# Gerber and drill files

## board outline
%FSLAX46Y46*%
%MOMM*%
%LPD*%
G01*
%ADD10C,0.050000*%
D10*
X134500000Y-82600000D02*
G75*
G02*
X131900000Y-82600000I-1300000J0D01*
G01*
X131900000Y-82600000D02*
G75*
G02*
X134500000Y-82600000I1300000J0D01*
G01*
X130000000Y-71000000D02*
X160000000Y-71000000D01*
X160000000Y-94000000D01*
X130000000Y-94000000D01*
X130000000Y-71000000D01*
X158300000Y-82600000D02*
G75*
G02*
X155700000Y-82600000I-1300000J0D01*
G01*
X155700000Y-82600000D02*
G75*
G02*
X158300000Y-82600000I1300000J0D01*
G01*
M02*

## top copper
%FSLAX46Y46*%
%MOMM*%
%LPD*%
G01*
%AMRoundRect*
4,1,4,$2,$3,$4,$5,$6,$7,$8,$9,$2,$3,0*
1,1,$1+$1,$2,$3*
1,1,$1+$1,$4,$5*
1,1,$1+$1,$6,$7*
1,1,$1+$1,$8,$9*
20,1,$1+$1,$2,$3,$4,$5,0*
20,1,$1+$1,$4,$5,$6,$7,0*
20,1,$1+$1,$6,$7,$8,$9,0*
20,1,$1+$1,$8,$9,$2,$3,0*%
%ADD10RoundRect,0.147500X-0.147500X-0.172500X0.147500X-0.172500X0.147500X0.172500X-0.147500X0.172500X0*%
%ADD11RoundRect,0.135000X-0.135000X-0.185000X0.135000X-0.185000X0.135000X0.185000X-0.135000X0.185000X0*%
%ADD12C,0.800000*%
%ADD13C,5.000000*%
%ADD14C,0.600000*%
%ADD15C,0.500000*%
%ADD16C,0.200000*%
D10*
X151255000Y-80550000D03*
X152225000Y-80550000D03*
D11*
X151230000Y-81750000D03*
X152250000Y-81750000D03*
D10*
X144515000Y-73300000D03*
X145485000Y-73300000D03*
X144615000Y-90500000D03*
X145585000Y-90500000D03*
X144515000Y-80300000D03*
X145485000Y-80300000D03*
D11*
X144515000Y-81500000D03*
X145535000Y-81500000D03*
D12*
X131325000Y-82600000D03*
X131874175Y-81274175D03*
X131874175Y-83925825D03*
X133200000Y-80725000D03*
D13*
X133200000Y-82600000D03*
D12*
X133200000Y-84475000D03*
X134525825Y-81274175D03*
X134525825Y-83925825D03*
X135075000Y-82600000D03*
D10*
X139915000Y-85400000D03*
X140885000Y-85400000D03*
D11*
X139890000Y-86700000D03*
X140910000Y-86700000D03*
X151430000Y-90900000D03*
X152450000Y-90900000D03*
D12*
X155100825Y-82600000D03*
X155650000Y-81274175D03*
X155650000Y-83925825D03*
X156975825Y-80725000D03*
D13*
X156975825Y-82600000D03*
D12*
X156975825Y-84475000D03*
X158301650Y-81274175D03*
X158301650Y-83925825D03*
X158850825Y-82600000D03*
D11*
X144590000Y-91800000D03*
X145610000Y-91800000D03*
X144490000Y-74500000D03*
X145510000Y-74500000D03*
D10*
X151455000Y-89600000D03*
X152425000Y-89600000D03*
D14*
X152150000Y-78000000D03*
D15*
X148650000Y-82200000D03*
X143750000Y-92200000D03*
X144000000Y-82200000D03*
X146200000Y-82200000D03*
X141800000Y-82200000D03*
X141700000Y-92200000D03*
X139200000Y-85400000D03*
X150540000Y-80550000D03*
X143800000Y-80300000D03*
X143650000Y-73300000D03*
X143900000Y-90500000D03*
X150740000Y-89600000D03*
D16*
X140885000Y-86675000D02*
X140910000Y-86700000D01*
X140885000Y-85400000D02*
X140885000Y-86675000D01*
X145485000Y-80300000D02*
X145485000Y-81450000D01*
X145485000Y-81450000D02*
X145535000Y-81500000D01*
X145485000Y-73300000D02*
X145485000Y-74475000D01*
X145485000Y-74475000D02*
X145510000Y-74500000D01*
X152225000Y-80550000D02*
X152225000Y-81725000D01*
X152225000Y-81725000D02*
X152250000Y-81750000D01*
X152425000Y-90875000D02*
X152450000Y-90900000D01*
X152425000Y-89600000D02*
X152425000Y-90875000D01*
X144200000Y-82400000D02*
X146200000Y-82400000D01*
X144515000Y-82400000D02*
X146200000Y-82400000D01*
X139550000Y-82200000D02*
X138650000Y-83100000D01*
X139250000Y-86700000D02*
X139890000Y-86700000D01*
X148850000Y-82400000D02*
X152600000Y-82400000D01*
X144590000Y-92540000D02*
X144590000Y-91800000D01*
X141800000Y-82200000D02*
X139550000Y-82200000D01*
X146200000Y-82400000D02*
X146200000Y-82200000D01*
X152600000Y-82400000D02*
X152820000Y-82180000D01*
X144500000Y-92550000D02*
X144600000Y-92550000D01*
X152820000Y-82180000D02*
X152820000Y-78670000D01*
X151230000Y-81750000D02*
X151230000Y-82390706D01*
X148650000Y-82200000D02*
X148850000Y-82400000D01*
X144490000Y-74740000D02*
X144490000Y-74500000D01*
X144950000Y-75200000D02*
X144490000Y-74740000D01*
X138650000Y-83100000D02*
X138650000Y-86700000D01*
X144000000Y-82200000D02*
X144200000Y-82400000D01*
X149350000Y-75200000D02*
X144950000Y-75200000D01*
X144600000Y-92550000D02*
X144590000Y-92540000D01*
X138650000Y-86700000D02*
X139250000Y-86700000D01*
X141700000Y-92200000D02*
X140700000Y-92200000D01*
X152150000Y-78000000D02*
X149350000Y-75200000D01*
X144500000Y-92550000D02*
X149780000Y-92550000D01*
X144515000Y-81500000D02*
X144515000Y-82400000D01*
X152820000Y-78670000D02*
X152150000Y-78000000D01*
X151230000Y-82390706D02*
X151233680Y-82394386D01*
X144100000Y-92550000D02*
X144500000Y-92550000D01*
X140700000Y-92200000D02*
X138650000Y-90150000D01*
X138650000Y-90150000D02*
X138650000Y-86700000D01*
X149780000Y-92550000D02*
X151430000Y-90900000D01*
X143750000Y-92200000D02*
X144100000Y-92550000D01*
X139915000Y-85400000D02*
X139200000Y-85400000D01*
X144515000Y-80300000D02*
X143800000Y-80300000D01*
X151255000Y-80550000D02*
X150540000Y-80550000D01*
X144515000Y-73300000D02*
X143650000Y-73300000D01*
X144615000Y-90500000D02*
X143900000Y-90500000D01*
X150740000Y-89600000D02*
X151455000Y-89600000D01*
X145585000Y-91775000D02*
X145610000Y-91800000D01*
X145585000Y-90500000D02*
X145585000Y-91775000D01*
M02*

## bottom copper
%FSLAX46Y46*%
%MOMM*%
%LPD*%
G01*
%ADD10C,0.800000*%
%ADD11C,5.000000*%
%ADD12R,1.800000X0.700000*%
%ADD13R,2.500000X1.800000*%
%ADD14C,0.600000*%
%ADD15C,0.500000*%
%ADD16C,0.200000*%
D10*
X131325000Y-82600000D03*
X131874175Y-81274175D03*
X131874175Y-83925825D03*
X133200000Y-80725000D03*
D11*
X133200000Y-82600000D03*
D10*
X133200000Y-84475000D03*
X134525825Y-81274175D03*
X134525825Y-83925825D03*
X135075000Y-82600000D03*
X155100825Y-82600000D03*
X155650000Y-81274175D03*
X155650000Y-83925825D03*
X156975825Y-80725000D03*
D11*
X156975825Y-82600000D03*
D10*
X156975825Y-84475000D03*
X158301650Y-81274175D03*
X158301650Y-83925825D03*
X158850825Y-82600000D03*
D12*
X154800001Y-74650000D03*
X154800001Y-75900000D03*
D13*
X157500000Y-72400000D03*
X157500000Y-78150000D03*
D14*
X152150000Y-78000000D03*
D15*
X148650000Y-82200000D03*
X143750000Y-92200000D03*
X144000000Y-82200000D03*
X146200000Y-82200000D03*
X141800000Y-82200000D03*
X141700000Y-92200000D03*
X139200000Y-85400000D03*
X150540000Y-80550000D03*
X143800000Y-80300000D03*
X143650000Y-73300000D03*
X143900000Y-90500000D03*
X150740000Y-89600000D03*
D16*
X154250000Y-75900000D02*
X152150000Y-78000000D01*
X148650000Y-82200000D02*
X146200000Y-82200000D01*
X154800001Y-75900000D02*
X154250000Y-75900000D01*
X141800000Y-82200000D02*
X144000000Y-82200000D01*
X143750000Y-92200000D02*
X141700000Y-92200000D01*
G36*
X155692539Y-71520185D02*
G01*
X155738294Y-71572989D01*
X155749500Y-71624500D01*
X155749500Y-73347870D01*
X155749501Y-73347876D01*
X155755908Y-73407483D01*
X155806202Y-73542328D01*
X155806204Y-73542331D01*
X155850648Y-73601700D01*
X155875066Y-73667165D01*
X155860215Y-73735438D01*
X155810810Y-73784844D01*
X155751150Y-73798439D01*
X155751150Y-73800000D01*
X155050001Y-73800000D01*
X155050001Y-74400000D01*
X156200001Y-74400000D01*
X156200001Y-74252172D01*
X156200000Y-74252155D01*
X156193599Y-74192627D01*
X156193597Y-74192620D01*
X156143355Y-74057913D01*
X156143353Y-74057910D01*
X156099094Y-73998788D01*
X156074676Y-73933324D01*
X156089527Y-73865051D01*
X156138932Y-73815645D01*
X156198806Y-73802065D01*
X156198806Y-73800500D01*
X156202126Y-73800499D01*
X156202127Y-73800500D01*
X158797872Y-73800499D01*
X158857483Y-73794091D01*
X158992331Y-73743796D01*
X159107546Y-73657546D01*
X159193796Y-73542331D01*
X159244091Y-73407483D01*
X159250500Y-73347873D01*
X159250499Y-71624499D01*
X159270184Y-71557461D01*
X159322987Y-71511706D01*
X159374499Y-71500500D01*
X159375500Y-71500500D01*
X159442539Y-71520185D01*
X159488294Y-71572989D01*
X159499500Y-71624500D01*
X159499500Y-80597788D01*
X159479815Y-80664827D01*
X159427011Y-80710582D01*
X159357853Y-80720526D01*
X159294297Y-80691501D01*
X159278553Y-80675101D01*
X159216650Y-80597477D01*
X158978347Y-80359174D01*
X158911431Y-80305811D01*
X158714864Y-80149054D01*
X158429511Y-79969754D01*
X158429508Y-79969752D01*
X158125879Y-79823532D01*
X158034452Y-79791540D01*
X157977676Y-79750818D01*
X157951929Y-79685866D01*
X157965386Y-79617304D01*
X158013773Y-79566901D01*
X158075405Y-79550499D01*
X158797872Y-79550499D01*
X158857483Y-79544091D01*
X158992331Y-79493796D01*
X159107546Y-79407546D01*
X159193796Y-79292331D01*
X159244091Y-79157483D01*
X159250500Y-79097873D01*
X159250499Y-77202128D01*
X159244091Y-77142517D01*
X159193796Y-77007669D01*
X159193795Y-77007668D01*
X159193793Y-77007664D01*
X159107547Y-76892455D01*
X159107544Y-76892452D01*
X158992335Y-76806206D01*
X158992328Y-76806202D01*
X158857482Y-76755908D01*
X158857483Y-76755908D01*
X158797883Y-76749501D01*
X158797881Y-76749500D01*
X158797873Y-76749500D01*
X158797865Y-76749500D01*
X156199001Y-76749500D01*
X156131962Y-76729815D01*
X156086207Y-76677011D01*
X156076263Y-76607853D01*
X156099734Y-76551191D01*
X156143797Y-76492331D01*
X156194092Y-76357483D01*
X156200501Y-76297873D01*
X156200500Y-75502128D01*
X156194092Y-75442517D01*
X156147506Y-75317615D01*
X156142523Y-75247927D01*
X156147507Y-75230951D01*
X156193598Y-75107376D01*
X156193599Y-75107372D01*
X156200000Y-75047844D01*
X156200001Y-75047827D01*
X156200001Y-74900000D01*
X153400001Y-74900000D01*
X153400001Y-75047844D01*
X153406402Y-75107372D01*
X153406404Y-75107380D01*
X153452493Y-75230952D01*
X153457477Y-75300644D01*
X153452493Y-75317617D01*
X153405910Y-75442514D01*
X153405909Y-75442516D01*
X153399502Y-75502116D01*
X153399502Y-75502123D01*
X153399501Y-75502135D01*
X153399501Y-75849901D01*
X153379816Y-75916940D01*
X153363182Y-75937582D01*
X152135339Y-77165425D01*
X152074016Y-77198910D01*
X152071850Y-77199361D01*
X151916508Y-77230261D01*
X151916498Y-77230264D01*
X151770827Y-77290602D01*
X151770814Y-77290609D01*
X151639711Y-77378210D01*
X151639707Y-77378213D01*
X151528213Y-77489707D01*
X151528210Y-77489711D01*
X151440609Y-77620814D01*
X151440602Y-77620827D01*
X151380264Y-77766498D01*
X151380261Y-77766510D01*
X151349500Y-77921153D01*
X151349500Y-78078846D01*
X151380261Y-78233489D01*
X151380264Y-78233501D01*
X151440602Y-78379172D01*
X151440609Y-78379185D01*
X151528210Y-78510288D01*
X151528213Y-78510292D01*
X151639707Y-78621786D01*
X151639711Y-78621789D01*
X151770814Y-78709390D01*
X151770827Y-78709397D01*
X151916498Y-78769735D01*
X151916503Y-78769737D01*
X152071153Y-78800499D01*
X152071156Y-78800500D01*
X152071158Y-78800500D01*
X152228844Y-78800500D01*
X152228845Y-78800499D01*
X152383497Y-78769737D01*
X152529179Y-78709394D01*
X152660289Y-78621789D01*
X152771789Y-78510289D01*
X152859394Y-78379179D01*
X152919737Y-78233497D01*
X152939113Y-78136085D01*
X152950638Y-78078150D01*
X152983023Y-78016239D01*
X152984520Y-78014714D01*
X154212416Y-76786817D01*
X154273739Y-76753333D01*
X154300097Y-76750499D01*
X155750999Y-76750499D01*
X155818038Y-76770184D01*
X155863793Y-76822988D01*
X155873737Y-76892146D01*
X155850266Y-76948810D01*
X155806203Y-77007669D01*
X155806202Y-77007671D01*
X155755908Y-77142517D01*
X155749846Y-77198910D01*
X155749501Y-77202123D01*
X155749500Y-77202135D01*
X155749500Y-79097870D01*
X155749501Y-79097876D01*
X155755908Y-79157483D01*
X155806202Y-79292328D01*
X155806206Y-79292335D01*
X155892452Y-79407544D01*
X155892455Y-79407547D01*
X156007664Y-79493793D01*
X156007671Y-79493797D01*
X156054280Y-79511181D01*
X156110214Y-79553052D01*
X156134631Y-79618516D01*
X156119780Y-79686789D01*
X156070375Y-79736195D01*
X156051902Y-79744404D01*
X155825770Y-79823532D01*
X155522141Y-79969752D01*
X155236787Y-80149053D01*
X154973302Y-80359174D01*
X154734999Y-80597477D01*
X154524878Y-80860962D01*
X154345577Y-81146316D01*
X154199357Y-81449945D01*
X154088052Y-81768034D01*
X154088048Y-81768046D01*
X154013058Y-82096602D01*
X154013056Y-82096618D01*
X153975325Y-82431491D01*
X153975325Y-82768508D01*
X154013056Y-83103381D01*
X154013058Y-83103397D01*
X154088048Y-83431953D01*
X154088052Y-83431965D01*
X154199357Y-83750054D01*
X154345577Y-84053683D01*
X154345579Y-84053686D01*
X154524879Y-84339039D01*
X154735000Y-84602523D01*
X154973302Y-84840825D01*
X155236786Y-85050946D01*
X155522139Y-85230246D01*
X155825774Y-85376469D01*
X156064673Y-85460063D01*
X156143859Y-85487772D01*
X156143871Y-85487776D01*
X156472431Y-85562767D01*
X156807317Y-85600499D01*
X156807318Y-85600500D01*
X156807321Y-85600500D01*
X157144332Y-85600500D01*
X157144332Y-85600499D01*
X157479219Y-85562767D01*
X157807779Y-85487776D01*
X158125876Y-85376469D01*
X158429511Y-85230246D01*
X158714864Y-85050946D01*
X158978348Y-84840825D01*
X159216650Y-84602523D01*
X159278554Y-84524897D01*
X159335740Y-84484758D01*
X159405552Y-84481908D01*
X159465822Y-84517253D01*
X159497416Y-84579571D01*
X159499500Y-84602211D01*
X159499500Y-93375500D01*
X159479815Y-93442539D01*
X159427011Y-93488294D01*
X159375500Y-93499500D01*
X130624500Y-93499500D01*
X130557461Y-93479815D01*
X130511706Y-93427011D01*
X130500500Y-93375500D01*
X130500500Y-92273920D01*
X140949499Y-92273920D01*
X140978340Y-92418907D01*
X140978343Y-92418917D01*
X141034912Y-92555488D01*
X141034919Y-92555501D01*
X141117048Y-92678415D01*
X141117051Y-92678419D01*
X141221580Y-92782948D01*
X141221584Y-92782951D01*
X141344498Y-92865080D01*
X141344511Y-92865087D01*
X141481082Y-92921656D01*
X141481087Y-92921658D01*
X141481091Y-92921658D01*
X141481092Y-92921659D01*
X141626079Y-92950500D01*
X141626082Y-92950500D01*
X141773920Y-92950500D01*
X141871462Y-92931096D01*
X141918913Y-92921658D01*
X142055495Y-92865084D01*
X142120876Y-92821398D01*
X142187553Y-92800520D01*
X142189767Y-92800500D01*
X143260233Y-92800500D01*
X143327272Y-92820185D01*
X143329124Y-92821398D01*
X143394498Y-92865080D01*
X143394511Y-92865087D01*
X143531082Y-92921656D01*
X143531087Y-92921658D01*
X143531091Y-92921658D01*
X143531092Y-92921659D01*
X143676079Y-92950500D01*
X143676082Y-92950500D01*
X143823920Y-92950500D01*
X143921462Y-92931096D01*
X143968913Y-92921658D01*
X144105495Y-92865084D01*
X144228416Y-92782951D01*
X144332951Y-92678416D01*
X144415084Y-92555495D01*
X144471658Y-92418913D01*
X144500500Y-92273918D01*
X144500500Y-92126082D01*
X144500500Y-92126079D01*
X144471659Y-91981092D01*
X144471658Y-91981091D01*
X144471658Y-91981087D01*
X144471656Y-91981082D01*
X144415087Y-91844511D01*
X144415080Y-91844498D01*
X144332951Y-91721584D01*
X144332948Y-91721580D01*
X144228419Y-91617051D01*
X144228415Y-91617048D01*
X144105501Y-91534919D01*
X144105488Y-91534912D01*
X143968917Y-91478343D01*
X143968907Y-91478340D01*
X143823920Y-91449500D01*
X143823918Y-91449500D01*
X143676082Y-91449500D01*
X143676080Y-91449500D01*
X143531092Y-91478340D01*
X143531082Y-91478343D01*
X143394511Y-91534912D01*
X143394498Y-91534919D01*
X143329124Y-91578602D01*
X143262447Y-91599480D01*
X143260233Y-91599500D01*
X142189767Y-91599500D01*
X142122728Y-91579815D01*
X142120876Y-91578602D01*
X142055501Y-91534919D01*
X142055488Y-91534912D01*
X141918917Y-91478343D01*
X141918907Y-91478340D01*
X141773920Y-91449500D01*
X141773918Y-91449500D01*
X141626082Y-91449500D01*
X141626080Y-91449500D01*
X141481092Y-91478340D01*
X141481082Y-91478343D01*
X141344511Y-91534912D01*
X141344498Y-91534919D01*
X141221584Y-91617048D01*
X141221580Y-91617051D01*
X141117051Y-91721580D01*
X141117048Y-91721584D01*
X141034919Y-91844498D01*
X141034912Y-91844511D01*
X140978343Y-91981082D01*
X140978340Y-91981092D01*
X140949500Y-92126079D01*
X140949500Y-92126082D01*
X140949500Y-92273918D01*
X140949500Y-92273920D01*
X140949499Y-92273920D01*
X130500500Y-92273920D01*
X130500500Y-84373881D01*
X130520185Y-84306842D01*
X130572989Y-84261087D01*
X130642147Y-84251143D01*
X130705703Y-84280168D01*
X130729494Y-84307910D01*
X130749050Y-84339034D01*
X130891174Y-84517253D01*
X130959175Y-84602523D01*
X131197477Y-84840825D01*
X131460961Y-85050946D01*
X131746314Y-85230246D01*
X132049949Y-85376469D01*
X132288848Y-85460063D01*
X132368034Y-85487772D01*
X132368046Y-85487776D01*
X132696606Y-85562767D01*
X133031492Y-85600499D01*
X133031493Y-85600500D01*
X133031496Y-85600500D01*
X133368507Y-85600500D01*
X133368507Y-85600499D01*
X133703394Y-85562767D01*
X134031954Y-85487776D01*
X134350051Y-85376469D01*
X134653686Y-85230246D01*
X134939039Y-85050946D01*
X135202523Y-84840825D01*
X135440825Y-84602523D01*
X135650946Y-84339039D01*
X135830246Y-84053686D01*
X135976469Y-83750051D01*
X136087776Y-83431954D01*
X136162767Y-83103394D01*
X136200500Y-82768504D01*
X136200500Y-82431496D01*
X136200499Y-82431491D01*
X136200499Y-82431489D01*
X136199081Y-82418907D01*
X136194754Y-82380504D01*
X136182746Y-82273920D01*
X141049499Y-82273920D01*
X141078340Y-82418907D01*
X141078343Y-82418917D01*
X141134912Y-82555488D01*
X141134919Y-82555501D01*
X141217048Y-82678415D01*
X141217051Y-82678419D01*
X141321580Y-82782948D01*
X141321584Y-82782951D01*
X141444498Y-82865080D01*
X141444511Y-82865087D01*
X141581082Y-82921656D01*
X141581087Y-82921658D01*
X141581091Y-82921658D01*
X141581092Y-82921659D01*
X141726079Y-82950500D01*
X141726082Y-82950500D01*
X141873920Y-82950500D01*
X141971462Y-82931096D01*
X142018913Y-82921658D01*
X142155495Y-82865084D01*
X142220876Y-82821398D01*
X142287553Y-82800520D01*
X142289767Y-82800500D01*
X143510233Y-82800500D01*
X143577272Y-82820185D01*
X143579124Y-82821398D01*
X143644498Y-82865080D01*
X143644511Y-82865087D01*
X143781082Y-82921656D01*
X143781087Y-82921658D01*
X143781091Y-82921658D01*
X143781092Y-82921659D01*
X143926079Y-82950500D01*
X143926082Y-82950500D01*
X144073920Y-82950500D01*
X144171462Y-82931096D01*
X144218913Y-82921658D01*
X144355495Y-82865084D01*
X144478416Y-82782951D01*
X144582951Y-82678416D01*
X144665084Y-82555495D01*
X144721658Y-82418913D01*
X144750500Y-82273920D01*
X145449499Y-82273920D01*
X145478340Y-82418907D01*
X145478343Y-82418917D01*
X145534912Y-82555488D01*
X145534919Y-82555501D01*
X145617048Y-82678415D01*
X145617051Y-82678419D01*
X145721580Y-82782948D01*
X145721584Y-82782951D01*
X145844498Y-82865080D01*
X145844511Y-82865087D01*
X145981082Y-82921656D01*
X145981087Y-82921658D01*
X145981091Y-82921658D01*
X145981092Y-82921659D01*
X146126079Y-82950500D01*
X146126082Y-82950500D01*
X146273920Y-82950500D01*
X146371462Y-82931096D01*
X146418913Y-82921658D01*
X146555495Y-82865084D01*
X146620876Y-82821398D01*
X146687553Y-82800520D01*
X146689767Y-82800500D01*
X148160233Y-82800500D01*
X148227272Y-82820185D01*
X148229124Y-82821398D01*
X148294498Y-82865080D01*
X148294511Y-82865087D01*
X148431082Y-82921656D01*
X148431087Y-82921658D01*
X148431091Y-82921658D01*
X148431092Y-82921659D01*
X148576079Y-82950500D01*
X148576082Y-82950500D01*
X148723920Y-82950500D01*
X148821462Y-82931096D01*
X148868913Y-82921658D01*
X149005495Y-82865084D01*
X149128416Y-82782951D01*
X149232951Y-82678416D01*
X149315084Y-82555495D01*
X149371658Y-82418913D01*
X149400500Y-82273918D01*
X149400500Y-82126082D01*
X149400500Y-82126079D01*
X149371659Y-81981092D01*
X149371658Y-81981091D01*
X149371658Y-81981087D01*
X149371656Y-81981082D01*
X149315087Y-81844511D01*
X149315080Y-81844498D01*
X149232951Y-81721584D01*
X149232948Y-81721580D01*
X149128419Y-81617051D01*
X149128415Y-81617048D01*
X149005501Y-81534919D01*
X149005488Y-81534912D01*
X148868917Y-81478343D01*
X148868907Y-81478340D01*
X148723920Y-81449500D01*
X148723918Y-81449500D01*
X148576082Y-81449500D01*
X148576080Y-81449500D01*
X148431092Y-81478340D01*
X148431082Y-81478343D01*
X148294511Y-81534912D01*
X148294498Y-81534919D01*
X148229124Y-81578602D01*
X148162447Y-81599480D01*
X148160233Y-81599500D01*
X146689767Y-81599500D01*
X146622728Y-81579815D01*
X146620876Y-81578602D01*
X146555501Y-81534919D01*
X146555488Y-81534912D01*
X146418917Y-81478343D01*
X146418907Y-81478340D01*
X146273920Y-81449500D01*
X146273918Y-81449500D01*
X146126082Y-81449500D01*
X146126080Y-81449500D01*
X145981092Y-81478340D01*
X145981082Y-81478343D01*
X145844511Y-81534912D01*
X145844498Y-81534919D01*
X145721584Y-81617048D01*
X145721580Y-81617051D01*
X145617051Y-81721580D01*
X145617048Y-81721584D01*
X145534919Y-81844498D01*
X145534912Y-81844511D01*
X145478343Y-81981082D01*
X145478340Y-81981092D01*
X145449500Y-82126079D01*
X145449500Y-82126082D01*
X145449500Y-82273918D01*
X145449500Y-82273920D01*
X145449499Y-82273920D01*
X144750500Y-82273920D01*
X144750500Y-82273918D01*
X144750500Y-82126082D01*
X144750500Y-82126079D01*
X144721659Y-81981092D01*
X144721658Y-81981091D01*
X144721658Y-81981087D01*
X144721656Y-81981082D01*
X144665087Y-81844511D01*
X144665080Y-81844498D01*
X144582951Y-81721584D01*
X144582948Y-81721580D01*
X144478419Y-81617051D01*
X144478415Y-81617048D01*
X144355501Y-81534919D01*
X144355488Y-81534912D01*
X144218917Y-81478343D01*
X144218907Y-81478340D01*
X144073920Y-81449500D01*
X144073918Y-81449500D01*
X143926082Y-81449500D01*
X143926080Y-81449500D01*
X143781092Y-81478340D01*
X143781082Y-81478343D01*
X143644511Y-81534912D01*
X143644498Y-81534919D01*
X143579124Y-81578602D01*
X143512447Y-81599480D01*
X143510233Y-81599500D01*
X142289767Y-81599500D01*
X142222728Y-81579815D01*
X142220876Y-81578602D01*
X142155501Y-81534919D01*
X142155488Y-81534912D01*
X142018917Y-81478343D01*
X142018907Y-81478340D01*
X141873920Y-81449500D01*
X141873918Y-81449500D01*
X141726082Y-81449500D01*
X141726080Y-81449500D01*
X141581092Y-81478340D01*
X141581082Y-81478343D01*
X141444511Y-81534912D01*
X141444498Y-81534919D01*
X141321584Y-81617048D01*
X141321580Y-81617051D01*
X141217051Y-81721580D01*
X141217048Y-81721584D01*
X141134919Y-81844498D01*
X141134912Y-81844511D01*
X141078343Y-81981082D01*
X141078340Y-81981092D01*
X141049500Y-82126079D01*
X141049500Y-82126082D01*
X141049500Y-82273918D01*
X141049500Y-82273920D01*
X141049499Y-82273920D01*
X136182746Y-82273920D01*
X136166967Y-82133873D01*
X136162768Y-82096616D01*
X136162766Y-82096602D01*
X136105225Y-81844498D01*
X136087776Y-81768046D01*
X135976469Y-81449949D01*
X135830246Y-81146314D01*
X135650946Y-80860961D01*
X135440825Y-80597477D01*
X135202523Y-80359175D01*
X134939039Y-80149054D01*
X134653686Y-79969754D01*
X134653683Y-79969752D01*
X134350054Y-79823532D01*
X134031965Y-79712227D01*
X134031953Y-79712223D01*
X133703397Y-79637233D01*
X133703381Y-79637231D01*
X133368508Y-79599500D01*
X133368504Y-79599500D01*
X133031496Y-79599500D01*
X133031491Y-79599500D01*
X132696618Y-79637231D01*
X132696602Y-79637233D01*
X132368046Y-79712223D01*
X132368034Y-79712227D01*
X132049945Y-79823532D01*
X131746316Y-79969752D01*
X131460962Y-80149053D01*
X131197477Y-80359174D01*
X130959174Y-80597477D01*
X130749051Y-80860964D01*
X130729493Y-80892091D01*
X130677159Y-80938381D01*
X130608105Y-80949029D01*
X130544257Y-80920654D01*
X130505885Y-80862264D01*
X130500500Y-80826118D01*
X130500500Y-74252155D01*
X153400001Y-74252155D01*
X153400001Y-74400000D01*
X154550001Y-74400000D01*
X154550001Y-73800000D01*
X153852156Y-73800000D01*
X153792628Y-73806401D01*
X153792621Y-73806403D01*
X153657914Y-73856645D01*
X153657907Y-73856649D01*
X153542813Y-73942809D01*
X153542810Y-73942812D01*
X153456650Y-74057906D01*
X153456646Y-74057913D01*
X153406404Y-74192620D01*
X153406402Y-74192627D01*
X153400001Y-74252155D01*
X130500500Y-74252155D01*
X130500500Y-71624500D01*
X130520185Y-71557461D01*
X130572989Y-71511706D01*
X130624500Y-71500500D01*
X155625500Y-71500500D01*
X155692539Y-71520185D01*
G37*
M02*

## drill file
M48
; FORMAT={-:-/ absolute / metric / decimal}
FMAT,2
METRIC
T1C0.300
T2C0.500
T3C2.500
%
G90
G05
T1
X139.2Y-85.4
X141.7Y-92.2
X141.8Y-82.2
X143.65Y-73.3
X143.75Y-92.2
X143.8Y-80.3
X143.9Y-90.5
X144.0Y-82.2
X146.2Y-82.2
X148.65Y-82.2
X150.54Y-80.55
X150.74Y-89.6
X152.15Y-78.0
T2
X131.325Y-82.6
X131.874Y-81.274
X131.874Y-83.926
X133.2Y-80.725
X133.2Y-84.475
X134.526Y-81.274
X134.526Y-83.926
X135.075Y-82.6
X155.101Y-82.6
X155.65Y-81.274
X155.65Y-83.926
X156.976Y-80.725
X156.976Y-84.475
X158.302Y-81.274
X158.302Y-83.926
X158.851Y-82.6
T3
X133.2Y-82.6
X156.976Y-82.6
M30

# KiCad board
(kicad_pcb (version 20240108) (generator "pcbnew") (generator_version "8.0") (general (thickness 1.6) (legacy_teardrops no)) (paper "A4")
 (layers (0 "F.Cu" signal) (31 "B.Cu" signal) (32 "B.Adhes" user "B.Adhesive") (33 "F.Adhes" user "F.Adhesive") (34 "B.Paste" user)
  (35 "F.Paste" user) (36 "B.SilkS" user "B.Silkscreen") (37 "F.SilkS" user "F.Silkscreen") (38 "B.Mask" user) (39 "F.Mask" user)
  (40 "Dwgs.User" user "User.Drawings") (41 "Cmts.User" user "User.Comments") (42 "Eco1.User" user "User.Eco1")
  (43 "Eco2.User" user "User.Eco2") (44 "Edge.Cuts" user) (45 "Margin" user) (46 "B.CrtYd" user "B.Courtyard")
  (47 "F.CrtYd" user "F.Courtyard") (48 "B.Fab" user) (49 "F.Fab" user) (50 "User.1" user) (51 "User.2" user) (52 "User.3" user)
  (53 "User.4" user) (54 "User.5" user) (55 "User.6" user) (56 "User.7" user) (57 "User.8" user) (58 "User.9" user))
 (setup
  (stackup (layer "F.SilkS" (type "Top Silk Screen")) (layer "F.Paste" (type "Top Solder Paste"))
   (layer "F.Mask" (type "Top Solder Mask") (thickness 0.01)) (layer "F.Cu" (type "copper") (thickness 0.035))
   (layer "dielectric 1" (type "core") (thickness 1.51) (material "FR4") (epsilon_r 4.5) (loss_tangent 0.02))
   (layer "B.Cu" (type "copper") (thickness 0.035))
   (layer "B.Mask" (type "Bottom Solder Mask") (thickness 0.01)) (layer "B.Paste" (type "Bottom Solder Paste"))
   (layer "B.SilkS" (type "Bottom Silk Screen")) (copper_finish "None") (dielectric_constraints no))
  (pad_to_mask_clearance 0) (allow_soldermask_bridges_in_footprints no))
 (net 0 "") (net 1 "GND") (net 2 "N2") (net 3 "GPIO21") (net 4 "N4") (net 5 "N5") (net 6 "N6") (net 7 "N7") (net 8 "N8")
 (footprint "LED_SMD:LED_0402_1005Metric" (layer "F.Cu") (at 151.74 80.55)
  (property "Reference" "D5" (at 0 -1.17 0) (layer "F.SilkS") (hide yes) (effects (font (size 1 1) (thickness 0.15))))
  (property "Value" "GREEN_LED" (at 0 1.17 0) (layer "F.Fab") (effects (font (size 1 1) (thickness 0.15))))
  (pad "1" smd roundrect (at -0.485 0) (size 0.59 0.64) (layers "F.Cu" "F.Paste" "F.Mask") (roundrect_rratio 0.25) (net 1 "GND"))
  (pad "2" smd roundrect (at 0.485 0) (size 0.59 0.64) (layers "F.Cu" "F.Paste" "F.Mask") (roundrect_rratio 0.25) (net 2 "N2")))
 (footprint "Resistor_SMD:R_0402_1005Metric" (layer "F.Cu") (at 151.74 81.75)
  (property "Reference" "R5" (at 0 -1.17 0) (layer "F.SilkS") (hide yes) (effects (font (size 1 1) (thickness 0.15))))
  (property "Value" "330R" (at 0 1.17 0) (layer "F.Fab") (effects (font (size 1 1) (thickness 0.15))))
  (pad "1" smd roundrect (at -0.51 0) (size 0.54 0.64) (layers "F.Cu" "F.Paste" "F.Mask") (roundrect_rratio 0.25) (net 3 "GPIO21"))
  (pad "2" smd roundrect (at 0.51 0) (size 0.54 0.64) (layers "F.Cu" "F.Paste" "F.Mask") (roundrect_rratio 0.25) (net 2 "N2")))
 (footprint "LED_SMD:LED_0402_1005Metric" (layer "F.Cu") (at 145 73.3)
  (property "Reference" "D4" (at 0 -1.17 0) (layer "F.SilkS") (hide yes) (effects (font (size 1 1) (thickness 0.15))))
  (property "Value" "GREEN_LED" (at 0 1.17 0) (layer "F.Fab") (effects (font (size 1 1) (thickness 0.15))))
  (pad "1" smd roundrect (at -0.485 0) (size 0.59 0.64) (layers "F.Cu" "F.Paste" "F.Mask") (roundrect_rratio 0.25) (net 1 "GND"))
  (pad "2" smd roundrect (at 0.485 0) (size 0.59 0.64) (layers "F.Cu" "F.Paste" "F.Mask") (roundrect_rratio 0.25) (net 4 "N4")))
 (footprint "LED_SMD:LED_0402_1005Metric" (layer "F.Cu") (at 145.1 90.5)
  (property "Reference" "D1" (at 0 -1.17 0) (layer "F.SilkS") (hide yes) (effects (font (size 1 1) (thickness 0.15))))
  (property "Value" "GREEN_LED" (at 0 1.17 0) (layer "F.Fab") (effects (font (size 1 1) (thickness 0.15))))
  (pad "1" smd roundrect (at -0.485 0) (size 0.59 0.64) (layers "F.Cu" "F.Paste" "F.Mask") (roundrect_rratio 0.25) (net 1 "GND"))
  (pad "2" smd roundrect (at 0.485 0) (size 0.59 0.64) (layers "F.Cu" "F.Paste" "F.Mask") (roundrect_rratio 0.25) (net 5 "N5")))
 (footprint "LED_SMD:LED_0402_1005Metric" (layer "F.Cu") (at 145 80.3)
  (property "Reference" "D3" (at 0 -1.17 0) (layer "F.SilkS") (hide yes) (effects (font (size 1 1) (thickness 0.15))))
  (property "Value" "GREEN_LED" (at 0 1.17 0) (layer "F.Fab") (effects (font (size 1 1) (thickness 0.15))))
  (pad "1" smd roundrect (at -0.485 0) (size 0.59 0.64) (layers "F.Cu" "F.Paste" "F.Mask") (roundrect_rratio 0.25) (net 1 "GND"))
  (pad "2" smd roundrect (at 0.485 0) (size 0.59 0.64) (layers "F.Cu" "F.Paste" "F.Mask") (roundrect_rratio 0.25) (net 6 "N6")))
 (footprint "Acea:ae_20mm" (layer "F.Cu") (at 144.822605 82.737829)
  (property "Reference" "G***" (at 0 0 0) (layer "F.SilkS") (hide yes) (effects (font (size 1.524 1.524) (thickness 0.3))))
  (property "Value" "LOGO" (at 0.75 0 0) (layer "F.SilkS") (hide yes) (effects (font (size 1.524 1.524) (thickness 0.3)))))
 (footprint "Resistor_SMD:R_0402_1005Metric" (layer "F.Cu") (at 145.025 81.5)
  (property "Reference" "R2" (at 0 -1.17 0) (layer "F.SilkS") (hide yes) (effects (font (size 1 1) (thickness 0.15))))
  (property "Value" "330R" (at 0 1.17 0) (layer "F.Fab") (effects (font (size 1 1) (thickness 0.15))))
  (pad "1" smd roundrect (at -0.51 0) (size 0.54 0.64) (layers "F.Cu" "F.Paste" "F.Mask") (roundrect_rratio 0.25) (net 3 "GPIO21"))
  (pad "2" smd roundrect (at 0.51 0) (size 0.54 0.64) (layers "F.Cu" "F.Paste" "F.Mask") (roundrect_rratio 0.25) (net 6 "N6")))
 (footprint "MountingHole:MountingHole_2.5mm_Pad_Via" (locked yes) (layer "F.Cu") (at 133.2 82.6)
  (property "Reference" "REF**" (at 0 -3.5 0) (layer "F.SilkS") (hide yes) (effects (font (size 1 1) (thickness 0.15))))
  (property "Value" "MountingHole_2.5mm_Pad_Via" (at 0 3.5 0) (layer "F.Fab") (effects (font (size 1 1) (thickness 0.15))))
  (pad "1" thru_hole circle (at -1.875 0) (size 0.8 0.8) (drill 0.5) (layers "*.Cu" "*.Mask") (remove_unused_layers no) (zone_connect 2))
  (pad "1" thru_hole circle (at -1.325825 -1.325825) (size 0.8 0.8) (drill 0.5) (layers "*.Cu" "*.Mask") (remove_unused_layers no)
   (zone_connect 2))
  (pad "1" thru_hole circle (at -1.325825 1.325825) (size 0.8 0.8) (drill 0.5) (layers "*.Cu" "*.Mask") (remove_unused_layers no)
   (zone_connect 2))
  (pad "1" thru_hole circle (at 0 -1.875) (size 0.8 0.8) (drill 0.5) (layers "*.Cu" "*.Mask") (remove_unused_layers no) (zone_connect 2))
  (pad "1" thru_hole circle (at 0 0) (size 5 5) (drill 2.5) (layers "*.Cu" "*.Mask") (remove_unused_layers no))
  (pad "1" thru_hole circle (at 0 1.875) (size 0.8 0.8) (drill 0.5) (layers "*.Cu" "*.Mask") (remove_unused_layers no) (zone_connect 2))
  (pad "1" thru_hole circle (at 1.325825 -1.325825) (size 0.8 0.8) (drill 0.5) (layers "*.Cu" "*.Mask") (remove_unused_layers no)
   (zone_connect 2))
  (pad "1" thru_hole circle (at 1.325825 1.325825) (size 0.8 0.8) (drill 0.5) (layers "*.Cu" "*.Mask") (remove_unused_layers no)
   (zone_connect 2))
  (pad "1" thru_hole circle (at 1.875 0) (size 0.8 0.8) (drill 0.5) (layers "*.Cu" "*.Mask") (remove_unused_layers no) (zone_connect 2)))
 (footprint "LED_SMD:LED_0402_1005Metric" (layer "F.Cu") (at 140.4 85.4)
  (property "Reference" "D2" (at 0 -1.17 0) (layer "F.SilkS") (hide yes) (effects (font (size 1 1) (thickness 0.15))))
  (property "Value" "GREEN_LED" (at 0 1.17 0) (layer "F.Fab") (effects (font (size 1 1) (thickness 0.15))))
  (pad "1" smd roundrect (at -0.485 0) (size 0.59 0.64) (layers "F.Cu" "F.Paste" "F.Mask") (roundrect_rratio 0.25) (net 1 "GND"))
  (pad "2" smd roundrect (at 0.485 0) (size 0.59 0.64) (layers "F.Cu" "F.Paste" "F.Mask") (roundrect_rratio 0.25) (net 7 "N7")))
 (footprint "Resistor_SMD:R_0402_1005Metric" (layer "F.Cu") (at 140.4 86.7)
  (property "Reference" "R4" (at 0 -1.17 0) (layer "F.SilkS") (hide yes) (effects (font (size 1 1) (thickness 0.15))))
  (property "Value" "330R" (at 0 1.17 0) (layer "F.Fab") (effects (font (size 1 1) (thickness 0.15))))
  (pad "1" smd roundrect (at -0.51 0) (size 0.54 0.64) (layers "F.Cu" "F.Paste" "F.Mask") (roundrect_rratio 0.25) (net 3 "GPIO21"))
  (pad "2" smd roundrect (at 0.51 0) (size 0.54 0.64) (layers "F.Cu" "F.Paste" "F.Mask") (roundrect_rratio 0.25) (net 7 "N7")))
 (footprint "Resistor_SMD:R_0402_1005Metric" (layer "F.Cu") (at 151.94 90.9)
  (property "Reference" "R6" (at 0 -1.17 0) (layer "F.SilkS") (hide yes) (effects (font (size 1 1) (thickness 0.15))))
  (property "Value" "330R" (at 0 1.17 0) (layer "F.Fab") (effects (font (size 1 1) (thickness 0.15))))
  (pad "1" smd roundrect (at -0.51 0) (size 0.54 0.64) (layers "F.Cu" "F.Paste" "F.Mask") (roundrect_rratio 0.25) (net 3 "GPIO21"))
  (pad "2" smd roundrect (at 0.51 0) (size 0.54 0.64) (layers "F.Cu" "F.Paste" "F.Mask") (roundrect_rratio 0.25) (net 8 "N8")))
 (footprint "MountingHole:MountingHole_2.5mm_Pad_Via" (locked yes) (layer "F.Cu") (at 156.975825 82.6)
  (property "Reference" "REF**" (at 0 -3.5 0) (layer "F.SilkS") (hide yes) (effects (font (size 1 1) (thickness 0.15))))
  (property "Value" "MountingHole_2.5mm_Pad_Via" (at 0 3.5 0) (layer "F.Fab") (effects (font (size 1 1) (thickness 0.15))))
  (pad "1" thru_hole circle (at -1.875 0) (size 0.8 0.8) (drill 0.5) (layers "*.Cu" "*.Mask") (remove_unused_layers no) (zone_connect 2))
  (pad "1" thru_hole circle (at -1.325825 -1.325825) (size 0.8 0.8) (drill 0.5) (layers "*.Cu" "*.Mask") (remove_unused_layers no)
   (zone_connect 2))
  (pad "1" thru_hole circle (at -1.325825 1.325825) (size 0.8 0.8) (drill 0.5) (layers "*.Cu" "*.Mask") (remove_unused_layers no)
   (zone_connect 2))
  (pad "1" thru_hole circle (at 0 -1.875) (size 0.8 0.8) (drill 0.5) (layers "*.Cu" "*.Mask") (remove_unused_layers no) (zone_connect 2))
  (pad "1" thru_hole circle (at 0 0) (size 5 5) (drill 2.5) (layers "*.Cu" "*.Mask") (remove_unused_layers no))
  (pad "1" thru_hole circle (at 0 1.875) (size 0.8 0.8) (drill 0.5) (layers "*.Cu" "*.Mask") (remove_unused_layers no) (zone_connect 2))
  (pad "1" thru_hole circle (at 1.325825 -1.325825) (size 0.8 0.8) (drill 0.5) (layers "*.Cu" "*.Mask") (remove_unused_layers no)
   (zone_connect 2))
  (pad "1" thru_hole circle (at 1.325825 1.325825) (size 0.8 0.8) (drill 0.5) (layers "*.Cu" "*.Mask") (remove_unused_layers no)
   (zone_connect 2))
  (pad "1" thru_hole circle (at 1.875 0) (size 0.8 0.8) (drill 0.5) (layers "*.Cu" "*.Mask") (remove_unused_layers no) (zone_connect 2)))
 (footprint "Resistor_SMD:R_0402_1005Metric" (layer "F.Cu") (at 145.1 91.8)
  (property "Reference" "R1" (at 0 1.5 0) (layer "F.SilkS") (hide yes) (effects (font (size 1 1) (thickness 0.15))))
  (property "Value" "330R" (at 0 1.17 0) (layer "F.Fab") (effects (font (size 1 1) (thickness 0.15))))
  (pad "1" smd roundrect (at -0.51 0) (size 0.54 0.64) (layers "F.Cu" "F.Paste" "F.Mask") (roundrect_rratio 0.25) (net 3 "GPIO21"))
  (pad "2" smd roundrect (at 0.51 0) (size 0.54 0.64) (layers "F.Cu" "F.Paste" "F.Mask") (roundrect_rratio 0.25) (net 5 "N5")))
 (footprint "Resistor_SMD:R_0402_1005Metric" (layer "F.Cu") (at 145 74.5)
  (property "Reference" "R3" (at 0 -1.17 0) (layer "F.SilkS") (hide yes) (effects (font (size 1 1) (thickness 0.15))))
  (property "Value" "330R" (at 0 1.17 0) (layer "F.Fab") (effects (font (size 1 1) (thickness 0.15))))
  (pad "1" smd roundrect (at -0.51 0) (size 0.54 0.64) (layers "F.Cu" "F.Paste" "F.Mask") (roundrect_rratio 0.25) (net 3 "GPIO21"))
  (pad "2" smd roundrect (at 0.51 0) (size 0.54 0.64) (layers "F.Cu" "F.Paste" "F.Mask") (roundrect_rratio 0.25) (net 4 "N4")))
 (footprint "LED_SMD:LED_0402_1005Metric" (layer "F.Cu") (at 151.94 89.6)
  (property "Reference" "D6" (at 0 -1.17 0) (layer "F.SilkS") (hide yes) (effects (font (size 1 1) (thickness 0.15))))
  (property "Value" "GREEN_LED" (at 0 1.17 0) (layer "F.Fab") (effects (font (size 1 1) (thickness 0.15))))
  (pad "1" smd roundrect (at -0.485 0) (size 0.59 0.64) (layers "F.Cu" "F.Paste" "F.Mask") (roundrect_rratio 0.25) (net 1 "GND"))
  (pad "2" smd roundrect (at 0.485 0) (size 0.59 0.64) (layers "F.Cu" "F.Paste" "F.Mask") (roundrect_rratio 0.25) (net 8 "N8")))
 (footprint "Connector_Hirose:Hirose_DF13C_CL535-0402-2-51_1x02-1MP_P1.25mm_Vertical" (layer "B.Cu") (at 156.250001 75.275 -90)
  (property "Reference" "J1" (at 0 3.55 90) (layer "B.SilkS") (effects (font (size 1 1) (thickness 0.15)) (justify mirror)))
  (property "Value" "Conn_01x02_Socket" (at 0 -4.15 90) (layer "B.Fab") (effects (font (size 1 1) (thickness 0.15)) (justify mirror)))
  (pad "1" smd rect (at -0.625 1.45 270) (size 0.7 1.8) (layers "B.Cu" "B.Paste" "B.Mask") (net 1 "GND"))
  (pad "2" smd rect (at 0.625 1.45 270) (size 0.7 1.8) (layers "B.Cu" "B.Paste" "B.Mask") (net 3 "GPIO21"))
  (pad "MP" smd rect (at -2.875 -1.249999 270) (size 1.8 2.5) (layers "B.Cu" "B.Paste" "B.Mask"))
  (pad "MP" smd rect (at 2.875 -1.249999 270) (size 1.8 2.5) (layers "B.Cu" "B.Paste" "B.Mask")))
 (gr_circle (center 133.2 82.6) (end 134.5 82.6) (stroke (width 0.05) (type default)) (fill none) (layer "Edge.Cuts"))
 (gr_rect (start 130 71) (end 160 94) (stroke (width 0.05) (type default)) (fill none) (layer "Edge.Cuts"))
 (gr_circle (center 157 82.6) (end 158.3 82.6) (stroke (width 0.05) (type default)) (fill none) (layer "Edge.Cuts"))
 (segment (start 140.885 86.675) (end 140.91 86.7) (width 0.2) (layer "F.Cu") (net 7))
 (segment (start 140.885 85.4) (end 140.885 86.675) (width 0.2) (layer "F.Cu") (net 7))
 (segment (start 145.485 80.3) (end 145.485 81.45) (width 0.2) (layer "F.Cu") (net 6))
 (segment (start 145.485 81.45) (end 145.535 81.5) (width 0.2) (layer "F.Cu") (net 6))
 (segment (start 145.485 73.3) (end 145.485 74.475) (width 0.2) (layer "F.Cu") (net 4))
 (segment (start 145.485 74.475) (end 145.51 74.5) (width 0.2) (layer "F.Cu") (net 4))
 (segment (start 152.225 80.55) (end 152.225 81.725) (width 0.2) (layer "F.Cu") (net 2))
 (segment (start 152.225 81.725) (end 152.25 81.75) (width 0.2) (layer "F.Cu") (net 2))
 (segment (start 152.425 90.875) (end 152.45 90.9) (width 0.2) (layer "F.Cu") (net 8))
 (segment (start 152.425 89.6) (end 152.425 90.875) (width 0.2) (layer "F.Cu") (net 8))
 (segment (start 144.2 82.4) (end 146.2 82.4) (width 0.2) (layer "F.Cu") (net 3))
 (segment (start 144.515 82.4) (end 146.2 82.4) (width 0.2) (layer "F.Cu") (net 3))
 (segment (start 139.55 82.2) (end 138.65 83.1) (width 0.2) (layer "F.Cu") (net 3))
 (segment (start 139.25 86.7) (end 139.89 86.7) (width 0.2) (layer "F.Cu") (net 3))
 (segment (start 148.85 82.4) (end 152.6 82.4) (width 0.2) (layer "F.Cu") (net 3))
 (segment (start 144.59 92.54) (end 144.59 91.8) (width 0.2) (layer "F.Cu") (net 3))
 (segment (start 141.8 82.2) (end 139.55 82.2) (width 0.2) (layer "F.Cu") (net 3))
 (segment (start 146.2 82.4) (end 146.2 82.2) (width 0.2) (layer "F.Cu") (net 3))
 (segment (start 152.6 82.4) (end 152.82 82.18) (width 0.2) (layer "F.Cu") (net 3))
 (segment (start 144.5 92.55) (end 144.6 92.55) (width 0.2) (layer "F.Cu") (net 3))
 (segment (start 152.82 82.18) (end 152.82 78.67) (width 0.2) (layer "F.Cu") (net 3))
 (segment (start 151.23 81.75) (end 151.23 82.390706) (width 0.2) (layer "F.Cu") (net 3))
 (segment (start 148.65 82.2) (end 148.85 82.4) (width 0.2) (layer "F.Cu") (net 3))
 (segment (start 144.49 74.74) (end 144.49 74.5) (width 0.2) (layer "F.Cu") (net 3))
 (segment (start 144.95 75.2) (end 144.49 74.74) (width 0.2) (layer "F.Cu") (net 3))
 (segment (start 138.65 83.1) (end 138.65 86.7) (width 0.2) (layer "F.Cu") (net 3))
 (segment (start 144 82.2) (end 144.2 82.4) (width 0.2) (layer "F.Cu") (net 3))
 (segment (start 149.35 75.2) (end 144.95 75.2) (width 0.2) (layer "F.Cu") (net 3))
 (segment (start 144.6 92.55) (end 144.59 92.54) (width 0.2) (layer "F.Cu") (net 3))
 (segment (start 138.65 86.7) (end 139.25 86.7) (width 0.2) (layer "F.Cu") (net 3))
 (segment (start 141.7 92.2) (end 140.7 92.2) (width 0.2) (layer "F.Cu") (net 3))
 (segment (start 152.15 78) (end 149.35 75.2) (width 0.2) (layer "F.Cu") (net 3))
 (segment (start 144.5 92.55) (end 149.78 92.55) (width 0.2) (layer "F.Cu") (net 3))
 (segment (start 144.515 81.5) (end 144.515 82.4) (width 0.2) (layer "F.Cu") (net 3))
 (segment (start 152.82 78.67) (end 152.15 78) (width 0.2) (layer "F.Cu") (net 3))
 (segment (start 151.23 82.390706) (end 151.23368 82.394386) (width 0.2) (layer "F.Cu") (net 3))
 (segment (start 144.1 92.55) (end 144.5 92.55) (width 0.2) (layer "F.Cu") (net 3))
 (segment (start 140.7 92.2) (end 138.65 90.15) (width 0.2) (layer "F.Cu") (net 3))
 (segment (start 138.65 90.15) (end 138.65 86.7) (width 0.2) (layer "F.Cu") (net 3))
 (segment (start 149.78 92.55) (end 151.43 90.9) (width 0.2) (layer "F.Cu") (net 3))
 (segment (start 143.75 92.2) (end 144.1 92.55) (width 0.2) (layer "F.Cu") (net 3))
 (via (at 152.15 78) (size 0.6) (drill 0.3) (layers "F.Cu" "B.Cu") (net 3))
 (via (at 148.65 82.2) (size 0.5) (drill 0.3) (layers "F.Cu" "B.Cu") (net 3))
 (via (at 143.75 92.2) (size 0.5) (drill 0.3) (layers "F.Cu" "B.Cu") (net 3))
 (via (at 144 82.2) (size 0.5) (drill 0.3) (layers "F.Cu" "B.Cu") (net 3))
 (via (at 146.2 82.2) (size 0.5) (drill 0.3) (layers "F.Cu" "B.Cu") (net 3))
 (via (at 141.8 82.2) (size 0.5) (drill 0.3) (layers "F.Cu" "B.Cu") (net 3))
 (via (at 141.7 92.2) (size 0.5) (drill 0.3) (layers "F.Cu" "B.Cu") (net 3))
 (segment (start 154.25 75.9) (end 152.15 78) (width 0.2) (layer "B.Cu") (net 3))
 (segment (start 148.65 82.2) (end 146.2 82.2) (width 0.2) (layer "B.Cu") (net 3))
 (segment (start 154.800001 75.9) (end 154.25 75.9) (width 0.2) (layer "B.Cu") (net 3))
 (segment (start 141.8 82.2) (end 144 82.2) (width 0.2) (layer "B.Cu") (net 3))
 (segment (start 143.75 92.2) (end 141.7 92.2) (width 0.2) (layer "B.Cu") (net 3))
 (segment (start 139.915 85.4) (end 139.2 85.4) (width 0.2) (layer "F.Cu") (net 1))
 (segment (start 144.515 80.3) (end 143.8 80.3) (width 0.2) (layer "F.Cu") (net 1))
 (segment (start 151.255 80.55) (end 150.54 80.55) (width 0.2) (layer "F.Cu") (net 1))
 (segment (start 144.515 73.3) (end 143.65 73.3) (width 0.2) (layer "F.Cu") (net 1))
 (segment (start 144.615 90.5) (end 143.9 90.5) (width 0.2) (layer "F.Cu") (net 1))
 (segment (start 150.74 89.6) (end 151.455 89.6) (width 0.2) (layer "F.Cu") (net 1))
 (via (at 139.2 85.4) (size 0.5) (drill 0.3) (layers "F.Cu" "B.Cu") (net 1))
 (via (at 150.54 80.55) (size 0.5) (drill 0.3) (layers "F.Cu" "B.Cu") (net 1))
 (via (at 143.8 80.3) (size 0.5) (drill 0.3) (layers "F.Cu" "B.Cu") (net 1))
 (via (at 143.65 73.3) (size 0.5) (drill 0.3) (layers "F.Cu" "B.Cu") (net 1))
 (via (at 143.9 90.5) (size 0.5) (drill 0.3) (layers "F.Cu" "B.Cu") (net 1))
 (via (at 150.74 89.6) (size 0.5) (drill 0.3) (layers "F.Cu" "B.Cu") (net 1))
 (segment (start 145.585 91.775) (end 145.61 91.8) (width 0.2) (layer "F.Cu") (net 5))
 (segment (start 145.585 90.5) (end 145.585 91.775) (width 0.2) (layer "F.Cu") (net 5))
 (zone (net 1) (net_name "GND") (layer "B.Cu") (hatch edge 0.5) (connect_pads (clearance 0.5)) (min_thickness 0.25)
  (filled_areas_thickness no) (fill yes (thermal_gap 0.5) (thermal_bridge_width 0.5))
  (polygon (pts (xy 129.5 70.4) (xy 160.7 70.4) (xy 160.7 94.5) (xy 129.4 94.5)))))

